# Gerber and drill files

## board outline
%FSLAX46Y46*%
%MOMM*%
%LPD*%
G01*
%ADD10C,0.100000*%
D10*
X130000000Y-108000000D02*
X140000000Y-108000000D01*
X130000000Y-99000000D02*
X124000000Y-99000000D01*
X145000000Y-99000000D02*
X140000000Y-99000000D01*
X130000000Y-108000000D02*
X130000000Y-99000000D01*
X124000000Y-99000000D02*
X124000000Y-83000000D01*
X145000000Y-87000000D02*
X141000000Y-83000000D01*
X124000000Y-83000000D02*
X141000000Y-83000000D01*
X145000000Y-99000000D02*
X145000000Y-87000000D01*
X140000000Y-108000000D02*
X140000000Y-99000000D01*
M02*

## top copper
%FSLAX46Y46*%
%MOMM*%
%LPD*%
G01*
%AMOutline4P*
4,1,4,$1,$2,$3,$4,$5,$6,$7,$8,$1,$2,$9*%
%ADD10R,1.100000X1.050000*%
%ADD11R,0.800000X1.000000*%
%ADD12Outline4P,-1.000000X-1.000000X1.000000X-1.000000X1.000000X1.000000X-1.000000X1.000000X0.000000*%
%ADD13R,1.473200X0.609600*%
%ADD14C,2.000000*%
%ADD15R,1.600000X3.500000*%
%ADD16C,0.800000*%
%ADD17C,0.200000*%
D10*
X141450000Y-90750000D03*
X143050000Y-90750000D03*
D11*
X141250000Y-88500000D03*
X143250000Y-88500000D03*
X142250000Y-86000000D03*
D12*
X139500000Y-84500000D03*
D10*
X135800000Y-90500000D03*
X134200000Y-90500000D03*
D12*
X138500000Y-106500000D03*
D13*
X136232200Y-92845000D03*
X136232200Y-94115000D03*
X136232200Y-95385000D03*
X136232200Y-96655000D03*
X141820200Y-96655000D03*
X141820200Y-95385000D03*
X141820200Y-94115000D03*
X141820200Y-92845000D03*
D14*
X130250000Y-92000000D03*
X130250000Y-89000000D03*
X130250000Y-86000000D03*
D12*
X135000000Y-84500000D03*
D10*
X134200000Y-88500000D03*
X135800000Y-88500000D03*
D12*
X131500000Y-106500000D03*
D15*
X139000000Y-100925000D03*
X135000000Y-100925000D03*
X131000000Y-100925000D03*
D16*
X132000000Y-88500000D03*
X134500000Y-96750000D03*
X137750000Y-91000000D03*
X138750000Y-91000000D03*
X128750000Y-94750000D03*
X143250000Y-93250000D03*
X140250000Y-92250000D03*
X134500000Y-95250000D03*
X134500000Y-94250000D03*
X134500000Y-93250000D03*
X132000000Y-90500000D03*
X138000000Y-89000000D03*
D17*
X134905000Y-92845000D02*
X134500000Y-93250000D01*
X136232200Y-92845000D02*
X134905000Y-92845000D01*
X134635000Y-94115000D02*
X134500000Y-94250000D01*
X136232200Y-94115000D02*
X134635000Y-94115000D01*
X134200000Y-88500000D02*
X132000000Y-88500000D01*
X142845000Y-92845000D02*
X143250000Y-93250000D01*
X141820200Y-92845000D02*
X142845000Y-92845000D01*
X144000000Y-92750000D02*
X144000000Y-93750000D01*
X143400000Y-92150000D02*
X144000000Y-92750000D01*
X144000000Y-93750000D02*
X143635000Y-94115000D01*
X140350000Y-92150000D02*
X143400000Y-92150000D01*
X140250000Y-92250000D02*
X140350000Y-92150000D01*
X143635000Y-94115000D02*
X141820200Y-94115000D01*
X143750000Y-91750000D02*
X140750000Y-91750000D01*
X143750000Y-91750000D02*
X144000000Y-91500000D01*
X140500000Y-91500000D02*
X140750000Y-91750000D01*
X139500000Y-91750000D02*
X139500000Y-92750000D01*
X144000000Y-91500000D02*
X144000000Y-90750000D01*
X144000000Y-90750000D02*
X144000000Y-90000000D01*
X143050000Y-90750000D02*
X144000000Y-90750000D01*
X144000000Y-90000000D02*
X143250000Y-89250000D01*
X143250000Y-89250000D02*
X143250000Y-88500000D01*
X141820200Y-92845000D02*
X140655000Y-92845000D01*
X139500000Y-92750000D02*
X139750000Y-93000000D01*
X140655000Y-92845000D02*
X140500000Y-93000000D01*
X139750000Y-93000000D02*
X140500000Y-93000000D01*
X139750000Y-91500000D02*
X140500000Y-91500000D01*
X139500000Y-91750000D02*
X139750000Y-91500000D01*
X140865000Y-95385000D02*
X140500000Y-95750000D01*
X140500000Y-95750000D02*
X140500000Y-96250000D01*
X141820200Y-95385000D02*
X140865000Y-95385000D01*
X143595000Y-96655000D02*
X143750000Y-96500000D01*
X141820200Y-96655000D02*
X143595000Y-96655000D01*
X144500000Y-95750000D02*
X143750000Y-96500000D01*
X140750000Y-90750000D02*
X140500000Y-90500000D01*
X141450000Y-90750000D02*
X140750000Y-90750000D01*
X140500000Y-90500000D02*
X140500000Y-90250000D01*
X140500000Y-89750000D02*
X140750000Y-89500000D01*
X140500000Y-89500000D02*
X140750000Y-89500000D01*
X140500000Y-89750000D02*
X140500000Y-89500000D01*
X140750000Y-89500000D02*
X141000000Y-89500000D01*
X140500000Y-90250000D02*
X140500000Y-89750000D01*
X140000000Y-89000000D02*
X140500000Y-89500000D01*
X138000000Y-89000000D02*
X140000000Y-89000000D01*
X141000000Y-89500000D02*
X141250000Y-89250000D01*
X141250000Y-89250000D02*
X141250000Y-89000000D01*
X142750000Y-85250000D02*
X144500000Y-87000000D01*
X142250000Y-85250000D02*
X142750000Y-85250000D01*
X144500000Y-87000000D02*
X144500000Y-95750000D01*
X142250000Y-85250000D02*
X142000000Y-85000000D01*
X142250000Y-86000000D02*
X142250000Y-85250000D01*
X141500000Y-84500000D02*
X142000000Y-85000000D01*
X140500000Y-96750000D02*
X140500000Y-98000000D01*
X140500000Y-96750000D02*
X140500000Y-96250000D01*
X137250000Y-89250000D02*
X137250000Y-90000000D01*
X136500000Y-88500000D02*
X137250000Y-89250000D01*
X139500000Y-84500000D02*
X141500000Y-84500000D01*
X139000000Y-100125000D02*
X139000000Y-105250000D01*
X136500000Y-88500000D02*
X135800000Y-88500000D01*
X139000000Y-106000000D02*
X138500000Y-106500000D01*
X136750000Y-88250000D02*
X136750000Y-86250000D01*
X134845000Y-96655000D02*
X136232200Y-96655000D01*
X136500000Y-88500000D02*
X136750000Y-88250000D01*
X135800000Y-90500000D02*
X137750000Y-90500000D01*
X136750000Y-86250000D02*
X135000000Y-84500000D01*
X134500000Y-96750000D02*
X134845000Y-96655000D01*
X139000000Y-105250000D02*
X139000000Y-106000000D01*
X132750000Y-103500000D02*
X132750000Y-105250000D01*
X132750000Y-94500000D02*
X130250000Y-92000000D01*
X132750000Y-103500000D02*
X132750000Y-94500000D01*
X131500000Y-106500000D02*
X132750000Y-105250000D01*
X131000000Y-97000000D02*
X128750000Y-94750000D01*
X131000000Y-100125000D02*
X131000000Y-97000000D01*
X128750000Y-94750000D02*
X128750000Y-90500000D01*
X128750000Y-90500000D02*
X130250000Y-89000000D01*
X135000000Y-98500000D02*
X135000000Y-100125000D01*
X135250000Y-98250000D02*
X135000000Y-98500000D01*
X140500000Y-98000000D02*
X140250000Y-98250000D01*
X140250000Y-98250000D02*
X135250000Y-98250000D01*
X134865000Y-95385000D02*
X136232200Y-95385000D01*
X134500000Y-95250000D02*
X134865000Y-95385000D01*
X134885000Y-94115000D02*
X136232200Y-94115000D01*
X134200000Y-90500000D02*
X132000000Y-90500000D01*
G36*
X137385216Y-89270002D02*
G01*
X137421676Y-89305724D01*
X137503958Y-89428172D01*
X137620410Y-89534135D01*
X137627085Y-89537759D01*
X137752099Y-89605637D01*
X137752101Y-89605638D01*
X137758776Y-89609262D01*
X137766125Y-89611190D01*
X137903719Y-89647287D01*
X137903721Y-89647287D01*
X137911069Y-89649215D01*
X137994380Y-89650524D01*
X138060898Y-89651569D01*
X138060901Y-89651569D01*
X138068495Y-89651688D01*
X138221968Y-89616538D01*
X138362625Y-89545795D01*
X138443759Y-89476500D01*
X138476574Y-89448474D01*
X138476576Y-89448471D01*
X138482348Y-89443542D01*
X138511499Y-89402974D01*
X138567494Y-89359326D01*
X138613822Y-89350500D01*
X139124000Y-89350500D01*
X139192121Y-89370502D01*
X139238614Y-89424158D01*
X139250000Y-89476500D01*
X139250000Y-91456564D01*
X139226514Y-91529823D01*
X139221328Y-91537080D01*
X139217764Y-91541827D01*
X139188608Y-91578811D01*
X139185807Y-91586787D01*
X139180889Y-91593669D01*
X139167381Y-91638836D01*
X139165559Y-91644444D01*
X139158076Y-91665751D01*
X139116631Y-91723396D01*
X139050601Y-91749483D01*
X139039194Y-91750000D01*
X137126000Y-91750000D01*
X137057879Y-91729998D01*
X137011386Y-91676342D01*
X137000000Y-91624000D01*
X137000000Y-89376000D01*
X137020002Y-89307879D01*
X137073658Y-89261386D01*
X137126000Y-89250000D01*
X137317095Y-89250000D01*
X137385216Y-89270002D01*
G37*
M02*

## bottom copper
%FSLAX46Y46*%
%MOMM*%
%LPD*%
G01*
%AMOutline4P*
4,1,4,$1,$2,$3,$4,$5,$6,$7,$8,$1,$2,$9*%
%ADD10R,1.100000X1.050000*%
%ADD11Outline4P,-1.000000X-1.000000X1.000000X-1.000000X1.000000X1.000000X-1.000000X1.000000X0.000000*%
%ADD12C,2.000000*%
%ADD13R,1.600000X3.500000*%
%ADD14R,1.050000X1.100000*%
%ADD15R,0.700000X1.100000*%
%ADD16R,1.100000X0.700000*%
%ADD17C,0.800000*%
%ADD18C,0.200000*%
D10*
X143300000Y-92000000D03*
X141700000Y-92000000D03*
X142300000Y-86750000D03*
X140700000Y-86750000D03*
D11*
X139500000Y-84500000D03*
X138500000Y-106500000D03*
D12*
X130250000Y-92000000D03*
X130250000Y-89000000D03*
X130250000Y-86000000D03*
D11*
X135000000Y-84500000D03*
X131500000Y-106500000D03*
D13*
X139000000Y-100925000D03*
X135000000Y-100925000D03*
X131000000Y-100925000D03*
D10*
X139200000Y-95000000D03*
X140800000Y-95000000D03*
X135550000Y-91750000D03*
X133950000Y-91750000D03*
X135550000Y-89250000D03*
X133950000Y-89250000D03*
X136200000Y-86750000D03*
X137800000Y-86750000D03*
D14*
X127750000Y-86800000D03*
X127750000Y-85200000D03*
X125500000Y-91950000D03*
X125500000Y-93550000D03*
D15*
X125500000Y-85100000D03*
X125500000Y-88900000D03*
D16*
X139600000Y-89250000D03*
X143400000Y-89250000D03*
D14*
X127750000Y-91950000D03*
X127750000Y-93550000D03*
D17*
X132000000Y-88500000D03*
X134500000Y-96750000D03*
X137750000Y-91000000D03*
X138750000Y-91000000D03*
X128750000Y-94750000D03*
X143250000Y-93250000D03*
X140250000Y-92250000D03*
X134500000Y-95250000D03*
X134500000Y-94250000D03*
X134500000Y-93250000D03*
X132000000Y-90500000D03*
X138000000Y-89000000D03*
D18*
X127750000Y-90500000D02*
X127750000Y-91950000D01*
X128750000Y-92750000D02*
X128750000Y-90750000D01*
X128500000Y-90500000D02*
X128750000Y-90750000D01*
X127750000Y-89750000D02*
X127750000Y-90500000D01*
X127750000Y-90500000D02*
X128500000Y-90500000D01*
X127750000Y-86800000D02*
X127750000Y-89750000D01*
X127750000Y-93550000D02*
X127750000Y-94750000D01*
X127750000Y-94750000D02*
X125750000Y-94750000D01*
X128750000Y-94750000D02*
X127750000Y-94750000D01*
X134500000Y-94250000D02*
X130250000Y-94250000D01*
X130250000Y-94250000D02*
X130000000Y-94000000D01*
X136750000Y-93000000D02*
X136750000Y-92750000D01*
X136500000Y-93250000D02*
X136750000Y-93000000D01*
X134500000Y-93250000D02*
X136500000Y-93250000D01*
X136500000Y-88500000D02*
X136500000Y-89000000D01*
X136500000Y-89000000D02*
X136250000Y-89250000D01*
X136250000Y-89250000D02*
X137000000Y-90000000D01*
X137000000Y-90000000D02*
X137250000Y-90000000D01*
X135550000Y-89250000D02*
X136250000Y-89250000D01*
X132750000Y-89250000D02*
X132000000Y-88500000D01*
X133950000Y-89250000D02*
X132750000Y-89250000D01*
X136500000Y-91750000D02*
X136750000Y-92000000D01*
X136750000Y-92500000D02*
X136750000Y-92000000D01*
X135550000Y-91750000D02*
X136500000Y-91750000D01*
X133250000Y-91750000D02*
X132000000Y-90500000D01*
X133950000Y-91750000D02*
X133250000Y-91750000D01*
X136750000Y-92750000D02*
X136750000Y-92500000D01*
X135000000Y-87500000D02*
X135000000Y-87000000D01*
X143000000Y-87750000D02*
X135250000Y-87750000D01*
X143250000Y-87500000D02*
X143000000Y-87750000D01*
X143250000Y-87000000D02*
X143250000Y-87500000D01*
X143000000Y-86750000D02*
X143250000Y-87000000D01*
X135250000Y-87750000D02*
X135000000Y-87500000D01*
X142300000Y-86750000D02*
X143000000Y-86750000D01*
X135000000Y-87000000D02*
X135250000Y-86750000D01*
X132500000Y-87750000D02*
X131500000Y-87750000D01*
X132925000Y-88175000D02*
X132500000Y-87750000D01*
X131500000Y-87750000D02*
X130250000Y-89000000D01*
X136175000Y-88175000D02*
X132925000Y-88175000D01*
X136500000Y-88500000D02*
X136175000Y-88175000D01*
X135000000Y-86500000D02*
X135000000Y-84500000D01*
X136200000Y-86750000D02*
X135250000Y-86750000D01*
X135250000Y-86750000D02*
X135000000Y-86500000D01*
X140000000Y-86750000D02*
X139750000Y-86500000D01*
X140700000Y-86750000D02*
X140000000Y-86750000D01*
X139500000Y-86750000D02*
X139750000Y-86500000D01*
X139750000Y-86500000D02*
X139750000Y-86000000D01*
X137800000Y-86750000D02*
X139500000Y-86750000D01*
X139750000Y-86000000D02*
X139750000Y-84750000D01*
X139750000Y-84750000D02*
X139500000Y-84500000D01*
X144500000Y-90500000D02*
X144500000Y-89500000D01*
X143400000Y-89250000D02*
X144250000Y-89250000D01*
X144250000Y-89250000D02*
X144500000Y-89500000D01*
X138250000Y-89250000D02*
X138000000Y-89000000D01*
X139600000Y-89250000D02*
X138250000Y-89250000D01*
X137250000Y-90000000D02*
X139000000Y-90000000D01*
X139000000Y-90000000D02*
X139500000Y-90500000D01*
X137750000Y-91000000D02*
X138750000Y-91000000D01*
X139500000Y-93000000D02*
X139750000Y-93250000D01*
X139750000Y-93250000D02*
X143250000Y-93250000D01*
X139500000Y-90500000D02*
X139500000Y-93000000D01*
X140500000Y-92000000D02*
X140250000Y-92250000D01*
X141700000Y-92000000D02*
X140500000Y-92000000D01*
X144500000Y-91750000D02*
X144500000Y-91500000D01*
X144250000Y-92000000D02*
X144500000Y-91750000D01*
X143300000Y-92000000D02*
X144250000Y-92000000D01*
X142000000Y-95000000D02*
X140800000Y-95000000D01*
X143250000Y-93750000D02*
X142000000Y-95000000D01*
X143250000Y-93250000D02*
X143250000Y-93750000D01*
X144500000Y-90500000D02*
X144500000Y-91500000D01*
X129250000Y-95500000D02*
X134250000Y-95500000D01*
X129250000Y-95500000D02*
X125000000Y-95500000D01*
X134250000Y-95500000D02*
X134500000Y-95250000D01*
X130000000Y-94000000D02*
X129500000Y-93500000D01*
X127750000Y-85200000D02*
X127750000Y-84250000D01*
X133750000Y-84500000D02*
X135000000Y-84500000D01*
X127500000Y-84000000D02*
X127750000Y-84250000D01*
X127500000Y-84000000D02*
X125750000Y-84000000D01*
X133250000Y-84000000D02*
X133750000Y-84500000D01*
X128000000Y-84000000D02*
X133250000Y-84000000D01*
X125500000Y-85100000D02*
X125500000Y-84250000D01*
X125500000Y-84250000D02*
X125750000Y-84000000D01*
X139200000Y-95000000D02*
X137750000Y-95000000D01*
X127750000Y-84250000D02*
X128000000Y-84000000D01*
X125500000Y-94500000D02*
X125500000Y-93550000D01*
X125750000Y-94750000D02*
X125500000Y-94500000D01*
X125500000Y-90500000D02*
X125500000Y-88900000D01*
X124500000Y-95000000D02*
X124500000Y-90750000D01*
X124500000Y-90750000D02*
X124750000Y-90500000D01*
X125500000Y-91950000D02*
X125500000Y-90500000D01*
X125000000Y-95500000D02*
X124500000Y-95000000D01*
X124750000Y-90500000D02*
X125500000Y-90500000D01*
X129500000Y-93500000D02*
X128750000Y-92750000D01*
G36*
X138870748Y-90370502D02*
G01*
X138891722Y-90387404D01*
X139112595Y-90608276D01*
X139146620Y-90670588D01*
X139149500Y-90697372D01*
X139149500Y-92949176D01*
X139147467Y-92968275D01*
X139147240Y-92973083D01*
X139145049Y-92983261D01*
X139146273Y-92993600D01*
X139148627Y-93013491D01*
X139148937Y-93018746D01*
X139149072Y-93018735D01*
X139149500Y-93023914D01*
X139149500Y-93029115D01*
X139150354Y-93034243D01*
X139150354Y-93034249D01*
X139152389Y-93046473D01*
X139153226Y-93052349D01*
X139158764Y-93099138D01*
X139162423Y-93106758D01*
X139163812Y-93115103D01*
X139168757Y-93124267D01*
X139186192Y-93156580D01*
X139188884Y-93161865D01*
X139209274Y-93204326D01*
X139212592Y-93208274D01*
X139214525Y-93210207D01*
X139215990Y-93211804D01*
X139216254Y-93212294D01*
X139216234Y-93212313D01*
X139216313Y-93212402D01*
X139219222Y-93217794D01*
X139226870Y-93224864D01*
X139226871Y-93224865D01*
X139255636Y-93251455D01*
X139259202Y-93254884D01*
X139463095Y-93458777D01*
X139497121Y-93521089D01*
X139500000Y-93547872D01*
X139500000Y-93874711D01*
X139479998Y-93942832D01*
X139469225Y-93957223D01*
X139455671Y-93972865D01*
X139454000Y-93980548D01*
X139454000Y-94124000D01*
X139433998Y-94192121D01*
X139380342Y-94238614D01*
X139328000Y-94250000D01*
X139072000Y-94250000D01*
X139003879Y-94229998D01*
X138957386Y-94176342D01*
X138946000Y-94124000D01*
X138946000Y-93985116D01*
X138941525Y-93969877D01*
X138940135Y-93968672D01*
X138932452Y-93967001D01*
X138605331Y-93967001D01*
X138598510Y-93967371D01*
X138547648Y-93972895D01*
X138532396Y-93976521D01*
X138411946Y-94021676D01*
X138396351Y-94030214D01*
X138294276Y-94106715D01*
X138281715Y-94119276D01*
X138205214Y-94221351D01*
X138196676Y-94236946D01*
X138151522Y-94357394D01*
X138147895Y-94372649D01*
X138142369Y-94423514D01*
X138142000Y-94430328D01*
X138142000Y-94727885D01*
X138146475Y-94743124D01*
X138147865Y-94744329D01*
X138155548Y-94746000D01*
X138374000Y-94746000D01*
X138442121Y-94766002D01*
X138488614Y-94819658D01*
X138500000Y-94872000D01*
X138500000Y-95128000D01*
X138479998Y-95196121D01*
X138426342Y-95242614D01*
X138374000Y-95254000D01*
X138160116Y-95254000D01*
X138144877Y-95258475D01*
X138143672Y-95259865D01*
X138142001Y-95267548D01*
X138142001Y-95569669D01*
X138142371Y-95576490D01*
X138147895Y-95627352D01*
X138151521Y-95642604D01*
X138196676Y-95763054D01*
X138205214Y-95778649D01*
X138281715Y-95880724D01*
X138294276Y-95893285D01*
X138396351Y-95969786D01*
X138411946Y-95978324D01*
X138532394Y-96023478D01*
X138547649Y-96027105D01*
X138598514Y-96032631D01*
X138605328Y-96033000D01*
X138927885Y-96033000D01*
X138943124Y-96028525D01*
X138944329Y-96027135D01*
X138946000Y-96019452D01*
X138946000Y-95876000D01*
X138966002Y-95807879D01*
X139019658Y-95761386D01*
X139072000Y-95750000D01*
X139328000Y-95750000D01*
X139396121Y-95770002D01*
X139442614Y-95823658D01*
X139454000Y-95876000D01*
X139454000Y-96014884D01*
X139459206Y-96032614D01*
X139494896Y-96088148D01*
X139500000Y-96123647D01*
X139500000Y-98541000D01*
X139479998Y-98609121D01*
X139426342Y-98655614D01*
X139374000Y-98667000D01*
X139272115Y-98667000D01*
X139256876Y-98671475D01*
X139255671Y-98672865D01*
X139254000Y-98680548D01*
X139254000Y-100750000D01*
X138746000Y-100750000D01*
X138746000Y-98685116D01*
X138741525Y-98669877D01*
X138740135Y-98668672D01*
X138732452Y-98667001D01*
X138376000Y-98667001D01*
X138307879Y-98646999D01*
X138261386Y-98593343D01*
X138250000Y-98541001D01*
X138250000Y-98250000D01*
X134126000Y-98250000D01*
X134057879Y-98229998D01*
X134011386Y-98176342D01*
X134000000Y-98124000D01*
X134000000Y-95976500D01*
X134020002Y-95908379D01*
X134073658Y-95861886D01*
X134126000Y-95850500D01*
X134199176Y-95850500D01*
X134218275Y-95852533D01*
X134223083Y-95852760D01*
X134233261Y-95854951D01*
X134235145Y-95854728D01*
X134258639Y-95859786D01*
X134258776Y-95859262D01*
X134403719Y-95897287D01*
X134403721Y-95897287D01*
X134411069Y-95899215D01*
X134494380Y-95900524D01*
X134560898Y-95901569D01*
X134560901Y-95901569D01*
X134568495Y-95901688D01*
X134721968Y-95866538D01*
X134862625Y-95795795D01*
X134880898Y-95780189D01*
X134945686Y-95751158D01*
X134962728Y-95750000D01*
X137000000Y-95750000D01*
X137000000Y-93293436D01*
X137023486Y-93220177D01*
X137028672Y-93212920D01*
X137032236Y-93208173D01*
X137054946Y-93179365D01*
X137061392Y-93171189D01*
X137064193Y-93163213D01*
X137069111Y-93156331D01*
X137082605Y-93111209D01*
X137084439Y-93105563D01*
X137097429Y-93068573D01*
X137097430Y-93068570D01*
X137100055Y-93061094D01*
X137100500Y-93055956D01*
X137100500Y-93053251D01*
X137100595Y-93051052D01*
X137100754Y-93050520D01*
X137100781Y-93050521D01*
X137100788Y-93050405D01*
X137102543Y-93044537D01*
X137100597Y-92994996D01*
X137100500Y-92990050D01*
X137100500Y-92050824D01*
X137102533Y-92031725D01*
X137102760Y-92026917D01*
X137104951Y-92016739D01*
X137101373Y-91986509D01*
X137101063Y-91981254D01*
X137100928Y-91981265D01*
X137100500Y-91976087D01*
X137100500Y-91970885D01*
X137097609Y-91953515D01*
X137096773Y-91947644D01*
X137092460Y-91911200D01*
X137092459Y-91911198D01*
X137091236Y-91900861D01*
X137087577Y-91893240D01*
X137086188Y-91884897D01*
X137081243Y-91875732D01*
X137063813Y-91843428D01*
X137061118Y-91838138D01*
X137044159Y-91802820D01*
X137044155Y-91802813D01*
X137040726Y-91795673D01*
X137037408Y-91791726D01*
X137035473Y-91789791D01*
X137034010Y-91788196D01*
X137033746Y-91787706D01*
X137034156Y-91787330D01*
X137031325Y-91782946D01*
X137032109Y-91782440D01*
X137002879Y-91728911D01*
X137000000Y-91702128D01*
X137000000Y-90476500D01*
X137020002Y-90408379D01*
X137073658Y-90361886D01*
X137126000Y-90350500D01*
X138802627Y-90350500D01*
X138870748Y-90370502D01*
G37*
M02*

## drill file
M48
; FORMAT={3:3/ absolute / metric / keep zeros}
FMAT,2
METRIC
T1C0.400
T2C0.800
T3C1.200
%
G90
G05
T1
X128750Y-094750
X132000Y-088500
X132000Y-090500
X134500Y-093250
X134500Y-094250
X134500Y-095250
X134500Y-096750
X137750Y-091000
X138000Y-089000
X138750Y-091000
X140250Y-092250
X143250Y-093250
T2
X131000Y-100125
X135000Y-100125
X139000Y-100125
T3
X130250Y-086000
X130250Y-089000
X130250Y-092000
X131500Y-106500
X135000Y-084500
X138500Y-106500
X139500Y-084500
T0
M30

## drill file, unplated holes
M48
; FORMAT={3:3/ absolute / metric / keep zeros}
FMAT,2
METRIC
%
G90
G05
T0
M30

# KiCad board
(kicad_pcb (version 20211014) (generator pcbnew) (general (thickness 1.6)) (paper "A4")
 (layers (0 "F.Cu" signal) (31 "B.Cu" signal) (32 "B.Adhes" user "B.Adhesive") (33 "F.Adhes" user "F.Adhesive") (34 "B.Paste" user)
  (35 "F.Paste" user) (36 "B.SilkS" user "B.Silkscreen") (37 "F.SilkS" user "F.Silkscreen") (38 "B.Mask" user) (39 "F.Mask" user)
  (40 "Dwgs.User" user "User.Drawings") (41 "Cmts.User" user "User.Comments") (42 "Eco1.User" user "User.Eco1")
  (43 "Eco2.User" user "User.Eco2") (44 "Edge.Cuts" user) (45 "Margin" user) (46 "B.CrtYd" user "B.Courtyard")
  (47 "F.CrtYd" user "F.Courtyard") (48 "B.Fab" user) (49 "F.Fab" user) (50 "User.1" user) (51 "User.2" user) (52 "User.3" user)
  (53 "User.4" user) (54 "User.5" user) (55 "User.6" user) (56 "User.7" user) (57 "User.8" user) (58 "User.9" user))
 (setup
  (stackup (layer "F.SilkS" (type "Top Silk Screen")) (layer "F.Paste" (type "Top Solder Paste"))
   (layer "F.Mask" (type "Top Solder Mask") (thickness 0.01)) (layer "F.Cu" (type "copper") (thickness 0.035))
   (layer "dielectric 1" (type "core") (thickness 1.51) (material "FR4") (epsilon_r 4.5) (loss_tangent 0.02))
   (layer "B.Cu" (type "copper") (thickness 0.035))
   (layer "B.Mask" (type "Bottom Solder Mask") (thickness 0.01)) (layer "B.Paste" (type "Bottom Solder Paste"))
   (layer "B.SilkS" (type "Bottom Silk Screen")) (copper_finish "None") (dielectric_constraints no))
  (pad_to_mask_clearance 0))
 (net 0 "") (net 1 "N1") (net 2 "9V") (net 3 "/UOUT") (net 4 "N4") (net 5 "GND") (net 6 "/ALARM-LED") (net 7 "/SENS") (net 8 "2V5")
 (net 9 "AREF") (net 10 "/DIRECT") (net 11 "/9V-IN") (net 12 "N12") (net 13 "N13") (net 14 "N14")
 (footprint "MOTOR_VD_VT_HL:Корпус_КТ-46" (layer "F.Cu") (at 142.25 87.25 90)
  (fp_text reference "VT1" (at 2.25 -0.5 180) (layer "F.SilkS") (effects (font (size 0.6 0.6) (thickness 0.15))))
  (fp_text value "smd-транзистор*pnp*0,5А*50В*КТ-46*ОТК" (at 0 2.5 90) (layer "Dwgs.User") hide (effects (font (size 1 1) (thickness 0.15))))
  (pad "1" smd rect locked (at -1.25 -1 90) (size 1 0.8) (layers "F.Cu" "F.Paste" "F.Mask") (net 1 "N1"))
  (pad "2" smd rect locked (at -1.25 1 90) (size 1 0.8) (layers "F.Cu" "F.Paste" "F.Mask") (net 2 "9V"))
  (pad "3" smd rect locked (at 1.25 0 90) (size 1 0.8) (layers "F.Cu" "F.Paste" "F.Mask") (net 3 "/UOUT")))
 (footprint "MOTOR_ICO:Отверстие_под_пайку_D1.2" (layer "F.Cu") (at 139.5 84.5)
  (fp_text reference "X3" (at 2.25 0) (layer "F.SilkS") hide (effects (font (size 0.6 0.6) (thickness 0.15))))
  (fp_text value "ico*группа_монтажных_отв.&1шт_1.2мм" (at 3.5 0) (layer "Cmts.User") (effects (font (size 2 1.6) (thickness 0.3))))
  (pad "1" thru_hole trapezoid locked (at 0 0) (size 2 2) (drill 1.2) (layers *.Cu *.Paste *.Mask) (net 3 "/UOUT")))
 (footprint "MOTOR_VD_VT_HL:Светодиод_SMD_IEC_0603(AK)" (layer "F.Cu") (at 135 90.5)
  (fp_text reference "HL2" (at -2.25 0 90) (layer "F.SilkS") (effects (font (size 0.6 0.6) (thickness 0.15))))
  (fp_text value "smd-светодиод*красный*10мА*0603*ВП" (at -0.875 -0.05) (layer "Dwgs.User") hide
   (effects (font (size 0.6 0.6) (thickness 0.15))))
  (pad "A" smd rect locked (at -0.8 0) (size 1.1 1.05) (layers "F.Cu" "F.Paste" "F.Mask") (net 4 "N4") (clearance 0.2))
  (pad "K" smd rect locked (at 0.8 0) (size 1.1 1.05) (layers "F.Cu" "F.Paste" "F.Mask") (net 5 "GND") (clearance 0.2)))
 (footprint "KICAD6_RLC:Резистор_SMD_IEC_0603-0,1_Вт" (layer "F.Cu") (at 142.25 90.75)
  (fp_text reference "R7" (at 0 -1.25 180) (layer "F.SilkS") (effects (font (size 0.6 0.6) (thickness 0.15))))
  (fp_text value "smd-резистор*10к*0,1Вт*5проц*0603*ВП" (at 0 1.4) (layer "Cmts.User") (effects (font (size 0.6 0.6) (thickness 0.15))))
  (pad "1" smd rect (at -0.8 0) (size 1.1 1.05) (layers "F.Cu" "F.Paste" "F.Mask") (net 1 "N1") (clearance 0.2))
  (pad "2" smd rect (at 0.8 0) (size 1.1 1.05) (layers "F.Cu" "F.Paste" "F.Mask") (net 2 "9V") (clearance 0.2)))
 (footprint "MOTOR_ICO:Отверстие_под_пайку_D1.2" (layer "F.Cu") (at 138.5 106.5)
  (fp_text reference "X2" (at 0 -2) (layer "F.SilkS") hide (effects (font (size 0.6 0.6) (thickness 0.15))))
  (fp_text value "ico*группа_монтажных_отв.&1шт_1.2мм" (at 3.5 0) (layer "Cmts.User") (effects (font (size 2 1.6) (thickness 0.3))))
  (pad "1" thru_hole trapezoid locked (at 0 0) (size 2 2) (drill 1.2) (layers *.Cu *.Paste *.Mask) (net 5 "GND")))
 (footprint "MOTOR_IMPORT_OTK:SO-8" (layer "F.Cu") (at 136.2682 92.861 -90)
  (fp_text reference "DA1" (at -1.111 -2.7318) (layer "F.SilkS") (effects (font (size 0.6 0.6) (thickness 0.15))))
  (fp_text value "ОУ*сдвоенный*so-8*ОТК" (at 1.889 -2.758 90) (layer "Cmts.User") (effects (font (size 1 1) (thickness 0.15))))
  (pad "1" smd rect locked (at -0.016 0.036 270) (size 0.6096 1.4732) (layers "F.Cu" "F.Paste" "F.Mask") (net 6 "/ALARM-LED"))
  (pad "2" smd rect locked (at 1.254 0.036 270) (size 0.6096 1.4732) (layers "F.Cu" "F.Paste" "F.Mask") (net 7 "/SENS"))
  (pad "3" smd rect locked (at 2.524 0.036 270) (size 0.6096 1.4732) (layers "F.Cu" "F.Paste" "F.Mask") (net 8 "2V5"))
  (pad "4" smd rect locked (at 3.794 0.036 270) (size 0.6096 1.4732) (layers "F.Cu" "F.Paste" "F.Mask") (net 5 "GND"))
  (pad "5" smd rect locked (at 3.794 -5.552 270) (size 0.6096 1.4732) (layers "F.Cu" "F.Paste" "F.Mask") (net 3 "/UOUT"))
  (pad "6" smd rect locked (at 2.524 -5.552 270) (size 0.6096 1.4732) (layers "F.Cu" "F.Paste" "F.Mask") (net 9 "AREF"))
  (pad "7" smd rect locked (at 1.254 -5.552 270) (size 0.6096 1.4732) (layers "F.Cu" "F.Paste" "F.Mask") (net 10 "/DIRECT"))
  (pad "8" smd rect locked (at -0.016 -5.552 270) (size 0.6096 1.4732) (layers "F.Cu" "F.Paste" "F.Mask") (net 2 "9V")))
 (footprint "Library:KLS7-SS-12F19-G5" (layer "F.Cu") (at 130.25 92 90)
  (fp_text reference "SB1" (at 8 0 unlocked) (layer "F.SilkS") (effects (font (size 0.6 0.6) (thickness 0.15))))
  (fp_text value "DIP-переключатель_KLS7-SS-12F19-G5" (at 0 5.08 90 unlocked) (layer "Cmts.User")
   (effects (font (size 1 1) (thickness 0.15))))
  (pad "1" thru_hole circle (at 0 0 90) (size 2 2) (drill 1.2) (layers *.Cu *.Mask) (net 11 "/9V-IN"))
  (pad "2" thru_hole circle (at 3 0 90) (size 2 2) (drill 1.2) (layers *.Cu *.Mask) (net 2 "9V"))
  (pad "3" thru_hole circle (at 6 0 90) (size 2 2) (drill 1.2) (layers *.Cu *.Mask) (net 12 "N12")))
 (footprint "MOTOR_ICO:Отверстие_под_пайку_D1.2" (layer "F.Cu") (at 135 84.5)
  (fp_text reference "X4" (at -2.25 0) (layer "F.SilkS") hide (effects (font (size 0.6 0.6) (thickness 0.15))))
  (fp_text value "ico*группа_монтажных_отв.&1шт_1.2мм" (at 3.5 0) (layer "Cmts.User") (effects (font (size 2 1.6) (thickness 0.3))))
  (pad "1" thru_hole trapezoid locked (at 0 0) (size 2 2) (drill 1.2) (layers *.Cu *.Paste *.Mask) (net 5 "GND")))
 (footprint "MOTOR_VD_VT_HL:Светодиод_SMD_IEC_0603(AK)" (layer "F.Cu") (at 135 88.5)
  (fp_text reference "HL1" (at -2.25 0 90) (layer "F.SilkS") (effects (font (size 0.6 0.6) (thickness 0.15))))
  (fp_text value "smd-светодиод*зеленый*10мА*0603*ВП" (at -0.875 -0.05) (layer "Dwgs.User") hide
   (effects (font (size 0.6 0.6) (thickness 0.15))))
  (pad "A" smd rect locked (at -0.8 0) (size 1.1 1.05) (layers "F.Cu" "F.Paste" "F.Mask") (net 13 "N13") (clearance 0.2))
  (pad "K" smd rect locked (at 0.8 0) (size 1.1 1.05) (layers "F.Cu" "F.Paste" "F.Mask") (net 5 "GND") (clearance 0.2)))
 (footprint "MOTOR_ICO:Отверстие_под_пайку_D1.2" (layer "F.Cu") (at 131.5 106.5)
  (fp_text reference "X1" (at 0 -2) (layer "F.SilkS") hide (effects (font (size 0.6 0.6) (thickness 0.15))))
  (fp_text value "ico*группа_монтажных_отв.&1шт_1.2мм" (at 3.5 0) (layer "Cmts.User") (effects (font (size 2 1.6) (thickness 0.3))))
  (pad "1" thru_hole trapezoid locked (at 0 0) (size 2 2) (drill 1.2) (layers *.Cu *.Paste *.Mask) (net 11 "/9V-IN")))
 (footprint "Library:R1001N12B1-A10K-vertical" (layer "F.Cu") (at 139 100.125 180)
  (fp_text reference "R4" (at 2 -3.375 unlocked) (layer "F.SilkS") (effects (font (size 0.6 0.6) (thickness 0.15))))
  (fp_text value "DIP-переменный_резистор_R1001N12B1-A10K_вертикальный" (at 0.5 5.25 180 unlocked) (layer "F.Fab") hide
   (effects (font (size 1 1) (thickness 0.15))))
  (pad "1" thru_hole rect (at 0 0 180) (size 1.6 3.5) (drill 0.8 (offset 0 -0.8)) (layers *.Cu *.Mask) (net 5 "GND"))
  (pad "2" thru_hole rect (at 4 0 180) (size 1.6 3.5) (drill 0.8 (offset 0 -0.8)) (layers *.Cu *.Mask) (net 9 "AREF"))
  (pad "3" thru_hole rect (at 8 0 180) (size 1.6 3.5) (drill 0.8 (offset 0 -0.8)) (layers *.Cu *.Mask) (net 2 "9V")))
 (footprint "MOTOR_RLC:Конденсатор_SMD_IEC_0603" (layer "B.Cu") (at 140 95)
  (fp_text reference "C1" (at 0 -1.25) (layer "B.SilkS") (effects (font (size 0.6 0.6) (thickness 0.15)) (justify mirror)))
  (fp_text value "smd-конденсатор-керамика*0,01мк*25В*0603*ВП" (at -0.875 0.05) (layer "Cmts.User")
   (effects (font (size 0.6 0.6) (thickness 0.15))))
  (pad "1" smd rect locked (at -0.8 0) (size 1.1 1.05) (layers "B.Cu" "B.Paste" "B.Mask") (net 5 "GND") (clearance 0.2))
  (pad "2" smd rect locked (at 0.8 0) (size 1.1 1.05) (layers "B.Cu" "B.Paste" "B.Mask") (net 2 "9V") (clearance 0.2)))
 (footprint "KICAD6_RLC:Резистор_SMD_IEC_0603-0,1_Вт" (layer "B.Cu") (at 134.75 91.75 180)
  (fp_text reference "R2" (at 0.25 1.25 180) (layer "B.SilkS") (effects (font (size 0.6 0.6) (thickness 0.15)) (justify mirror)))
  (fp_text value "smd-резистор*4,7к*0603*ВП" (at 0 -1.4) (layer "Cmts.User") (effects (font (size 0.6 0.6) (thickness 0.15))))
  (pad "1" smd rect (at -0.8 0 180) (size 1.1 1.05) (layers "B.Cu" "B.Paste" "B.Mask") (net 6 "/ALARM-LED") (clearance 0.2))
  (pad "2" smd rect (at 0.8 0 180) (size 1.1 1.05) (layers "B.Cu" "B.Paste" "B.Mask") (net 4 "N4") (clearance 0.2)))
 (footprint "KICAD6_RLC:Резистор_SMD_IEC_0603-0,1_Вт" (layer "B.Cu") (at 134.75 89.25 180)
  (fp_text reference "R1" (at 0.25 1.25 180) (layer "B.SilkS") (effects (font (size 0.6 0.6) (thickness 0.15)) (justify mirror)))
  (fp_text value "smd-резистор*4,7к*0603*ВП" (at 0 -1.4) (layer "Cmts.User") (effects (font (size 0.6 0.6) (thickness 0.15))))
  (pad "1" smd rect (at -0.8 0 180) (size 1.1 1.05) (layers "B.Cu" "B.Paste" "B.Mask") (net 2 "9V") (clearance 0.2))
  (pad "2" smd rect (at 0.8 0 180) (size 1.1 1.05) (layers "B.Cu" "B.Paste" "B.Mask") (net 13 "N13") (clearance 0.2)))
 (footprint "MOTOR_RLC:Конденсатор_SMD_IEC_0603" (layer "B.Cu") (at 137 86.75)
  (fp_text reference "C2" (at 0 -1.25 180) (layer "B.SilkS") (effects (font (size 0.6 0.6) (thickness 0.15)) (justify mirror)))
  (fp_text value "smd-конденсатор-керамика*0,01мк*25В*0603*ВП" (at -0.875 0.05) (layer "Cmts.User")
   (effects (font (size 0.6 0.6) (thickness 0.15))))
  (pad "1" smd rect locked (at -0.8 0) (size 1.1 1.05) (layers "B.Cu" "B.Paste" "B.Mask") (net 5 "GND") (clearance 0.2))
  (pad "2" smd rect locked (at 0.8 0) (size 1.1 1.05) (layers "B.Cu" "B.Paste" "B.Mask") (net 3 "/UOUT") (clearance 0.2)))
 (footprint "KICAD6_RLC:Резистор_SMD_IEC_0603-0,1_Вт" (layer "B.Cu") (at 127.75 86 -90)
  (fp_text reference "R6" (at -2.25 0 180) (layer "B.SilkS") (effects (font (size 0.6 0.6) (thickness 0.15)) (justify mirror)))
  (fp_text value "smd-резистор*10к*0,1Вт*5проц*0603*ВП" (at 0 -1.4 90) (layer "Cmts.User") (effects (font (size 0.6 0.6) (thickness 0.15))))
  (pad "1" smd rect (at -0.8 0 270) (size 1.1 1.05) (layers "B.Cu" "B.Paste" "B.Mask") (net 5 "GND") (clearance 0.2))
  (pad "2" smd rect (at 0.8 0 270) (size 1.1 1.05) (layers "B.Cu" "B.Paste" "B.Mask") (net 7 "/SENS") (clearance 0.2)))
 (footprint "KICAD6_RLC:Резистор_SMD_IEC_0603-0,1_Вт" (layer "B.Cu") (at 142.5 92 180)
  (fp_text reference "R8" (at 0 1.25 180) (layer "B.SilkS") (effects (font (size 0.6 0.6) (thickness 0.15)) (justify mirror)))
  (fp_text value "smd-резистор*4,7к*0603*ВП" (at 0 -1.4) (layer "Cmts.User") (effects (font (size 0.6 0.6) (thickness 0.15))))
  (pad "1" smd rect (at -0.8 0 180) (size 1.1 1.05) (layers "B.Cu" "B.Paste" "B.Mask") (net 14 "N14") (clearance 0.2))
  (pad "2" smd rect (at 0.8 0 180) (size 1.1 1.05) (layers "B.Cu" "B.Paste" "B.Mask") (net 10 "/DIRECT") (clearance 0.2)))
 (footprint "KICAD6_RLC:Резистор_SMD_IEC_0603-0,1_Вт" (layer "B.Cu") (at 125.5 92.75 -90)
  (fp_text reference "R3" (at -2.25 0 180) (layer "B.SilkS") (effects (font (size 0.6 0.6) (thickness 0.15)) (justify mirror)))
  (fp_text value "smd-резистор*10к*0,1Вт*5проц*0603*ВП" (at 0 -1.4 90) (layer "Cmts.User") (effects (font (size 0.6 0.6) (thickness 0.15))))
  (pad "1" smd rect (at -0.8 0 270) (size 1.1 1.05) (layers "B.Cu" "B.Paste" "B.Mask") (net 8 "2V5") (clearance 0.2))
  (pad "2" smd rect (at 0.8 0 270) (size 1.1 1.05) (layers "B.Cu" "B.Paste" "B.Mask") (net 2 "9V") (clearance 0.2)))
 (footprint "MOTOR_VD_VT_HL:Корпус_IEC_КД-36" (layer "B.Cu") (at 125.5 87 90)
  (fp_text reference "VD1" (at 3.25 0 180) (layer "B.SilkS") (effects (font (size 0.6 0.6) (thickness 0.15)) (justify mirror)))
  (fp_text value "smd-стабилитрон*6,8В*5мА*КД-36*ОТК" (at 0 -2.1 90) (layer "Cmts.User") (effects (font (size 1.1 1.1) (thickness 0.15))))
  (pad "A" smd rect locked (at 1.9 0 90) (size 1.1 0.7) (layers "B.Cu" "B.Paste" "B.Mask") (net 5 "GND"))
  (pad "K" smd rect locked (at -1.9 0 90) (size 1.1 0.7) (layers "B.Cu" "B.Paste" "B.Mask") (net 8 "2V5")))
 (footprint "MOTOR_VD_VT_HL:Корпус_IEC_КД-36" (layer "B.Cu") (at 141.5 89.25)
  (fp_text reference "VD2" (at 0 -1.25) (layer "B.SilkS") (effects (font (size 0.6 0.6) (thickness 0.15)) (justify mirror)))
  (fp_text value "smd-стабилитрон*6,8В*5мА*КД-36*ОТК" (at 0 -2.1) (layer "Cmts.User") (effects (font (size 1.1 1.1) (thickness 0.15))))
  (pad "A" smd rect locked (at 1.9 0) (size 1.1 0.7) (layers "B.Cu" "B.Paste" "B.Mask") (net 14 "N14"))
  (pad "K" smd rect locked (at -1.9 0) (size 1.1 0.7) (layers "B.Cu" "B.Paste" "B.Mask") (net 1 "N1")))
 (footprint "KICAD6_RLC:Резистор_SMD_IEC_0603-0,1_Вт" (layer "B.Cu") (at 141.5 86.75 180)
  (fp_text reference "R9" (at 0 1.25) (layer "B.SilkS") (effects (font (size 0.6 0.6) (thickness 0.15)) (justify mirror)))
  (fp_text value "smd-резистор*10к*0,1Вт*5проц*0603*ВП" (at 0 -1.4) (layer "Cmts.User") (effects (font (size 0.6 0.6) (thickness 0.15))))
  (pad "1" smd rect (at -0.8 0 180) (size 1.1 1.05) (layers "B.Cu" "B.Paste" "B.Mask") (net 5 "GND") (clearance 0.2))
  (pad "2" smd rect (at 0.8 0 180) (size 1.1 1.05) (layers "B.Cu" "B.Paste" "B.Mask") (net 3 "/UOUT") (clearance 0.2)))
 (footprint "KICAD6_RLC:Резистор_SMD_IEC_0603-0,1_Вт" (layer "B.Cu") (at 127.75 92.75 -90)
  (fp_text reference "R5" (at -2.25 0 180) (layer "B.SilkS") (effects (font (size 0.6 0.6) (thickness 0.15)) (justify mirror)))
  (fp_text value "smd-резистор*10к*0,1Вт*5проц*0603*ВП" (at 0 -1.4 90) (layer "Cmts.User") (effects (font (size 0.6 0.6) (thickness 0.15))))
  (pad "1" smd rect (at -0.8 0 270) (size 1.1 1.05) (layers "B.Cu" "B.Paste" "B.Mask") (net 7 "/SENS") (clearance 0.2))
  (pad "2" smd rect (at 0.8 0 270) (size 1.1 1.05) (layers "B.Cu" "B.Paste" "B.Mask") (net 2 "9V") (clearance 0.2)))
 (gr_line (start 130 108) (end 140 108) (layer "Edge.Cuts") (width 0.1))
 (gr_line (start 130 99) (end 124 99) (layer "Edge.Cuts") (width 0.1))
 (gr_line (start 145 99) (end 140 99) (layer "Edge.Cuts") (width 0.1))
 (gr_line (start 130 108) (end 130 99) (layer "Edge.Cuts") (width 0.1))
 (gr_line (start 124 99) (end 124 83) (layer "Edge.Cuts") (width 0.1))
 (gr_line (start 145 87) (end 141 83) (layer "Edge.Cuts") (width 0.1))
 (gr_line (start 124 83) (end 141 83) (layer "Edge.Cuts") (width 0.1))
 (gr_line (start 145 99) (end 145 87) (layer "Edge.Cuts") (width 0.1))
 (gr_line (start 140 108) (end 140 99) (layer "Edge.Cuts") (width 0.1))
 (segment (start 139 100.125) (end 139 105.25) (width 0.2) (layer "F.Cu") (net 5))
 (segment (start 136.5 88.5) (end 135.8 88.5) (width 0.2) (layer "F.Cu") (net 5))
 (segment (start 139 106) (end 138.5 106.5) (width 0.2) (layer "F.Cu") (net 5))
 (segment (start 136.75 88.25) (end 136.75 86.25) (width 0.2) (layer "F.Cu") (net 5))
 (segment (start 136.5 88.5) (end 137.25 89.25) (width 0.2) (layer "F.Cu") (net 5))
 (segment (start 134.845 96.655) (end 136.2322 96.655) (width 0.2) (layer "F.Cu") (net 5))
 (segment (start 136.5 88.5) (end 136.75 88.25) (width 0.2) (layer "F.Cu") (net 5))
 (segment (start 137.25 89.25) (end 137.25 90) (width 0.2) (layer "F.Cu") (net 5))
 (segment (start 135.8 90.5) (end 137.75 90.5) (width 0.2) (layer "F.Cu") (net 5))
 (segment (start 136.75 86.25) (end 135 84.5) (width 0.2) (layer "F.Cu") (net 5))
 (segment (start 134.5 96.75) (end 134.845 96.655) (width 0.2) (layer "F.Cu") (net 5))
 (segment (start 139 105.25) (end 139 106) (width 0.2) (layer "F.Cu") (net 5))
 (via (at 134.5 96.75) (size 0.8) (drill 0.4) (layers "F.Cu" "B.Cu") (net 5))
 (via (at 137.75 91) (size 0.8) (drill 0.4) (layers "F.Cu" "B.Cu") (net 5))
 (via (at 138.75 91) (size 0.8) (drill 0.4) (layers "F.Cu" "B.Cu") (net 5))
 (segment (start 127.75 85.2) (end 127.75 84.25) (width 0.2) (layer "B.Cu") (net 5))
 (segment (start 133.75 84.5) (end 135 84.5) (width 0.2) (layer "B.Cu") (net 5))
 (segment (start 143.25 87.5) (end 143 87.75) (width 0.2) (layer "B.Cu") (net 5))
 (segment (start 127.5 84) (end 127.75 84.25) (width 0.2) (layer "B.Cu") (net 5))
 (segment (start 143.25 87) (end 143.25 87.5) (width 0.2) (layer "B.Cu") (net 5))
 (segment (start 127.5 84) (end 125.75 84) (width 0.2) (layer "B.Cu") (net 5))
 (segment (start 135 87.5) (end 135 87) (width 0.2) (layer "B.Cu") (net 5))
 (segment (start 142.3 86.75) (end 143 86.75) (width 0.2) (layer "B.Cu") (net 5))
 (segment (start 133.25 84) (end 133.75 84.5) (width 0.2) (layer "B.Cu") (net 5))
 (segment (start 128 84) (end 133.25 84) (width 0.2) (layer "B.Cu") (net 5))
 (segment (start 136.2 86.75) (end 135.25 86.75) (width 0.2) (layer "B.Cu") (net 5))
 (segment (start 125.5 85.1) (end 125.5 84.25) (width 0.2) (layer "B.Cu") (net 5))
 (segment (start 143 86.75) (end 143.25 87) (width 0.2) (layer "B.Cu") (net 5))
 (segment (start 125.5 84.25) (end 125.75 84) (width 0.2) (layer "B.Cu") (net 5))
 (segment (start 139.2 95) (end 137.75 95) (width 0.2) (layer "B.Cu") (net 5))
 (segment (start 127.75 84.25) (end 128 84) (width 0.2) (layer "B.Cu") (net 5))
 (segment (start 135.25 86.75) (end 135 86.5) (width 0.2) (layer "B.Cu") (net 5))
 (segment (start 137.75 91) (end 138.75 91) (width 0.2) (layer "B.Cu") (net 5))
 (segment (start 135 86.5) (end 135 84.5) (width 0.2) (layer "B.Cu") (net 5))
 (segment (start 143 87.75) (end 135.25 87.75) (width 0.2) (layer "B.Cu") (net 5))
 (segment (start 135 87) (end 135.25 86.75) (width 0.2) (layer "B.Cu") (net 5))
 (segment (start 135.25 87.75) (end 135 87.5) (width 0.2) (layer "B.Cu") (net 5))
 (segment (start 132.75 103.5) (end 132.75 105.25) (width 0.2) (layer "F.Cu") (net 11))
 (segment (start 132.75 94.5) (end 130.25 92) (width 0.2) (layer "F.Cu") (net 11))
 (segment (start 132.75 103.5) (end 132.75 94.5) (width 0.2) (layer "F.Cu") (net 11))
 (segment (start 131.5 106.5) (end 132.75 105.25) (width 0.2) (layer "F.Cu") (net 11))
 (segment (start 134.2 88.5) (end 132 88.5) (width 0.2) (layer "F.Cu") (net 13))
 (via (at 132 88.5) (size 0.8) (drill 0.4) (layers "F.Cu" "B.Cu") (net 13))
 (segment (start 132.75 89.25) (end 132 88.5) (width 0.2) (layer "B.Cu") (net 13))
 (segment (start 133.95 89.25) (end 132.75 89.25) (width 0.2) (layer "B.Cu") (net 13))
 (segment (start 139.5 92.75) (end 139.75 93) (width 0.2) (layer "F.Cu") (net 2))
 (segment (start 131 97) (end 128.75 94.75) (width 0.2) (layer "F.Cu") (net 2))
 (segment (start 140.5 91.5) (end 140.75 91.75) (width 0.2) (layer "F.Cu") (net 2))
 (segment (start 139.5 91.75) (end 139.75 91.5) (width 0.2) (layer "F.Cu") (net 2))
 (segment (start 143.75 91.75) (end 144 91.5) (width 0.2) (layer "F.Cu") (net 2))
 (segment (start 144 91.5) (end 144 90.75) (width 0.2) (layer "F.Cu") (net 2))
 (segment (start 142.845 92.845) (end 143.25 93.25) (width 0.2) (layer "F.Cu") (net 2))
 (segment (start 139.75 91.5) (end 140.5 91.5) (width 0.2) (layer "F.Cu") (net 2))
 (segment (start 143.75 91.75) (end 140.75 91.75) (width 0.2) (layer "F.Cu") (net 2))
 (segment (start 131 100.125) (end 131 97) (width 0.2) (layer "F.Cu") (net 2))
 (segment (start 128.75 94.75) (end 128.75 90.5) (width 0.2) (layer "F.Cu") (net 2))
 (segment (start 140.655 92.845) (end 140.5 93) (width 0.2) (layer "F.Cu") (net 2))
 (segment (start 128.75 90.5) (end 130.25 89) (width 0.2) (layer "F.Cu") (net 2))
 (segment (start 143.25 89.25) (end 143.25 88.5) (width 0.2) (layer "F.Cu") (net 2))
 (segment (start 139.5 91.75) (end 139.5 92.75) (width 0.2) (layer "F.Cu") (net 2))
 (segment (start 141.8202 92.845) (end 140.655 92.845) (width 0.2) (layer "F.Cu") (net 2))
 (segment (start 139.75 93) (end 140.5 93) (width 0.2) (layer "F.Cu") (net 2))
 (segment (start 144 90) (end 143.25 89.25) (width 0.2) (layer "F.Cu") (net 2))
 (segment (start 143.05 90.75) (end 144 90.75) (width 0.2) (layer "F.Cu") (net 2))
 (segment (start 141.8202 92.845) (end 142.845 92.845) (width 0.2) (layer "F.Cu") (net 2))
 (segment (start 144 90.75) (end 144 90) (width 0.2) (layer "F.Cu") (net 2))
 (via (at 128.75 94.75) (size 0.8) (drill 0.4) (layers "F.Cu" "B.Cu") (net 2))
 (via (at 143.25 93.25) (size 0.8) (drill 0.4) (layers "F.Cu" "B.Cu") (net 2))
 (segment (start 139 90) (end 139.5 90.5) (width 0.2) (layer "B.Cu") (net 2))
 (segment (start 127.75 94.75) (end 125.75 94.75) (width 0.2) (layer "B.Cu") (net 2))
 (segment (start 125.5 94.5) (end 125.5 93.55) (width 0.2) (layer "B.Cu") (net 2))
 (segment (start 136.175 88.175) (end 132.925 88.175) (width 0.2) (layer "B.Cu") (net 2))
 (segment (start 125.75 94.75) (end 125.5 94.5) (width 0.2) (layer "B.Cu") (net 2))
 (segment (start 137 90) (end 137.25 90) (width 0.2) (layer "B.Cu") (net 2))
 (segment (start 136.25 89.25) (end 137 90) (width 0.2) (layer "B.Cu") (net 2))
 (segment (start 143.25 93.25) (end 143.25 93.75) (width 0.2) (layer "B.Cu") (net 2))
 (segment (start 132.925 88.175) (end 132.5 87.75) (width 0.2) (layer "B.Cu") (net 2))
 (segment (start 142 95) (end 140.8 95) (width 0.2) (layer "B.Cu") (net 2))
 (segment (start 139.75 93.25) (end 143.25 93.25) (width 0.2) (layer "B.Cu") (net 2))
 (segment (start 139.5 93) (end 139.75 93.25) (width 0.2) (layer "B.Cu") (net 2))
 (segment (start 136.5 88.5) (end 136.5 89) (width 0.2) (layer "B.Cu") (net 2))
 (segment (start 137.25 90) (end 139 90) (width 0.2) (layer "B.Cu") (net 2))
 (segment (start 128.75 94.75) (end 127.75 94.75) (width 0.2) (layer "B.Cu") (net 2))
 (segment (start 139.5 90.5) (end 139.5 93) (width 0.2) (layer "B.Cu") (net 2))
 (segment (start 135.55 89.25) (end 136.25 89.25) (width 0.2) (layer "B.Cu") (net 2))
 (segment (start 136.5 89) (end 136.25 89.25) (width 0.2) (layer "B.Cu") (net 2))
 (segment (start 143.25 93.75) (end 142 95) (width 0.2) (layer "B.Cu") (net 2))
 (segment (start 136.5 88.5) (end 136.175 88.175) (width 0.2) (layer "B.Cu") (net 2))
 (segment (start 132.5 87.75) (end 131.5 87.75) (width 0.2) (layer "B.Cu") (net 2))
 (segment (start 127.75 93.55) (end 127.75 94.75) (width 0.2) (layer "B.Cu") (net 2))
 (segment (start 131.5 87.75) (end 130.25 89) (width 0.2) (layer "B.Cu") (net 2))
 (segment (start 144.5 87) (end 144.5 95.75) (width 0.2) (layer "F.Cu") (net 3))
 (segment (start 139.5 84.5) (end 141.5 84.5) (width 0.2) (layer "F.Cu") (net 3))
 (segment (start 142.75 85.25) (end 144.5 87) (width 0.2) (layer "F.Cu") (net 3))
 (segment (start 142.25 86) (end 142.25 85.25) (width 0.2) (layer "F.Cu") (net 3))
 (segment (start 144.5 95.75) (end 143.75 96.5) (width 0.2) (layer "F.Cu") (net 3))
 (segment (start 141.5 84.5) (end 142 85) (width 0.2) (layer "F.Cu") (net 3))
 (segment (start 142.25 85.25) (end 142 85) (width 0.2) (layer "F.Cu") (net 3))
 (segment (start 142.25 85.25) (end 142.75 85.25) (width 0.2) (layer "F.Cu") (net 3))
 (segment (start 141.8202 96.655) (end 143.595 96.655) (width 0.2) (layer "F.Cu") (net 3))
 (segment (start 143.595 96.655) (end 143.75 96.5) (width 0.2) (layer "F.Cu") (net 3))
 (segment (start 140 86.75) (end 139.75 86.5) (width 0.2) (layer "B.Cu") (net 3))
 (segment (start 139.75 84.75) (end 139.5 84.5) (width 0.2) (layer "B.Cu") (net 3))
 (segment (start 139.5 86.75) (end 139.75 86.5) (width 0.2) (layer "B.Cu") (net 3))
 (segment (start 139.75 86.5) (end 139.75 86) (width 0.2) (layer "B.Cu") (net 3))
 (segment (start 139.75 86) (end 139.75 84.75) (width 0.2) (layer "B.Cu") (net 3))
 (segment (start 137.8 86.75) (end 139.5 86.75) (width 0.2) (layer "B.Cu") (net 3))
 (segment (start 140.7 86.75) (end 140 86.75) (width 0.2) (layer "B.Cu") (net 3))
 (segment (start 143.4 92.15) (end 144 92.75) (width 0.2) (layer "F.Cu") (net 10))
 (segment (start 143.635 94.115) (end 141.8202 94.115) (width 0.2) (layer "F.Cu") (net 10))
 (segment (start 140.35 92.15) (end 143.4 92.15) (width 0.2) (layer "F.Cu") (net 10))
 (segment (start 144 92.75) (end 144 93.75) (width 0.2) (layer "F.Cu") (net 10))
 (segment (start 144 93.75) (end 143.635 94.115) (width 0.2) (layer "F.Cu") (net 10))
 (segment (start 140.25 92.25) (end 140.35 92.15) (width 0.2) (layer "F.Cu") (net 10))
 (via (at 140.25 92.25) (size 0.8) (drill 0.4) (layers "F.Cu" "B.Cu") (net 10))
 (segment (start 140.5 92) (end 140.25 92.25) (width 0.2) (layer "B.Cu") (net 10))
 (segment (start 141.7 92) (end 140.5 92) (width 0.2) (layer "B.Cu") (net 10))
 (segment (start 140.5 96.75) (end 140.5 96.25) (width 0.2) (layer "F.Cu") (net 9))
 (segment (start 140.865 95.385) (end 140.5 95.75) (width 0.2) (layer "F.Cu") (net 9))
 (segment (start 135 98.5) (end 135 100.125) (width 0.2) (layer "F.Cu") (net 9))
 (segment (start 140.5 95.75) (end 140.5 96.25) (width 0.2) (layer "F.Cu") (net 9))
 (segment (start 135.25 98.25) (end 135 98.5) (width 0.2) (layer "F.Cu") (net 9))
 (segment (start 140.5 98) (end 140.25 98.25) (width 0.2) (layer "F.Cu") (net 9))
 (segment (start 141.8202 95.385) (end 140.865 95.385) (width 0.2) (layer "F.Cu") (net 9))
 (segment (start 140.25 98.25) (end 135.25 98.25) (width 0.2) (layer "F.Cu") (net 9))
 (segment (start 140.5 96.75) (end 140.5 98) (width 0.2) (layer "F.Cu") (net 9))
 (segment (start 134.865 95.385) (end 136.2322 95.385) (width 0.2) (layer "F.Cu") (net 8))
 (segment (start 134.5 95.25) (end 134.865 95.385) (width 0.2) (layer "F.Cu") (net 8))
 (via (at 134.5 95.25) (size 0.8) (drill 0.4) (layers "F.Cu" "B.Cu") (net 8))
 (segment (start 134.25 95.5) (end 134.5 95.25) (width 0.2) (layer "B.Cu") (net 8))
 (segment (start 125.5 90.5) (end 125.5 88.9) (width 0.2) (layer "B.Cu") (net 8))
 (segment (start 124.5 95) (end 124.5 90.75) (width 0.2) (layer "B.Cu") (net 8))
 (segment (start 124.5 90.75) (end 124.75 90.5) (width 0.2) (layer "B.Cu") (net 8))
 (segment (start 125.5 91.95) (end 125.5 90.5) (width 0.2) (layer "B.Cu") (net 8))
 (segment (start 125 95.5) (end 124.5 95) (width 0.2) (layer "B.Cu") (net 8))
 (segment (start 129.25 95.5) (end 125 95.5) (width 0.2) (layer "B.Cu") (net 8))
 (segment (start 124.75 90.5) (end 125.5 90.5) (width 0.2) (layer "B.Cu") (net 8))
 (segment (start 129.25 95.5) (end 134.25 95.5) (width 0.2) (layer "B.Cu") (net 8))
 (segment (start 134.635 94.115) (end 134.5 94.25) (width 0.2) (layer "F.Cu") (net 7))
 (segment (start 134.885 94.115) (end 136.2322 94.115) (width 0.2) (layer "F.Cu") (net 7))
 (segment (start 136.2322 94.115) (end 134.635 94.115) (width 0.2) (layer "F.Cu") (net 7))
 (via (at 134.5 94.25) (size 0.8) (drill 0.4) (layers "F.Cu" "B.Cu") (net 7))
 (segment (start 130.25 94.25) (end 130 94) (width 0.2) (layer "B.Cu") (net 7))
 (segment (start 128.5 90.5) (end 128.75 90.75) (width 0.2) (layer "B.Cu") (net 7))
 (segment (start 129.5 93.5) (end 128.75 92.75) (width 0.2) (layer "B.Cu") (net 7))
 (segment (start 127.75 90.5) (end 128.5 90.5) (width 0.2) (layer "B.Cu") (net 7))
 (segment (start 127.75 89.75) (end 127.75 90.5) (width 0.2) (layer "B.Cu") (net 7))
 (segment (start 130 94) (end 129.5 93.5) (width 0.2) (layer "B.Cu") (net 7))
 (segment (start 128.75 92.75) (end 128.75 90.75) (width 0.2) (layer "B.Cu") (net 7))
 (segment (start 127.75 90.5) (end 127.75 91.95) (width 0.2) (layer "B.Cu") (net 7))
 (segment (start 134.5 94.25) (end 130.25 94.25) (width 0.2) (layer "B.Cu") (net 7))
 (segment (start 127.75 86.8) (end 127.75 89.75) (width 0.2) (layer "B.Cu") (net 7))
 (segment (start 134.905 92.845) (end 134.5 93.25) (width 0.2) (layer "F.Cu") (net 6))
 (segment (start 136.2322 92.845) (end 134.905 92.845) (width 0.2) (layer "F.Cu") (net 6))
 (via (at 134.5 93.25) (size 0.8) (drill 0.4) (layers "F.Cu" "B.Cu") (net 6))
 (segment (start 136.75 93) (end 136.75 92.75) (width 0.2) (layer "B.Cu") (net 6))
 (segment (start 136.5 91.75) (end 136.75 92) (width 0.2) (layer "B.Cu") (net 6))
 (segment (start 136.5 93.25) (end 136.75 93) (width 0.2) (layer "B.Cu") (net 6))
 (segment (start 134.5 93.25) (end 136.5 93.25) (width 0.2) (layer "B.Cu") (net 6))
 (segment (start 135.55 91.75) (end 136.5 91.75) (width 0.2) (layer "B.Cu") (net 6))
 (segment (start 136.75 92.5) (end 136.75 92) (width 0.2) (layer "B.Cu") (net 6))
 (segment (start 136.75 92.75) (end 136.75 92.5) (width 0.2) (layer "B.Cu") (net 6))
 (segment (start 134.2 90.5) (end 132 90.5) (width 0.2) (layer "F.Cu") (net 4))
 (via (at 132 90.5) (size 0.8) (drill 0.4) (layers "F.Cu" "B.Cu") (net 4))
 (segment (start 133.25 91.75) (end 132 90.5) (width 0.2) (layer "B.Cu") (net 4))
 (segment (start 133.95 91.75) (end 133.25 91.75) (width 0.2) (layer "B.Cu") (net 4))
 (segment (start 141 89.5) (end 141.25 89.25) (width 0.2) (layer "F.Cu") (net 1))
 (segment (start 140.5 89.75) (end 140.75 89.5) (width 0.2) (layer "F.Cu") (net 1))
 (segment (start 138 89) (end 140 89) (width 0.2) (layer "F.Cu") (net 1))
 (segment (start 140.5 89.5) (end 140.75 89.5) (width 0.2) (layer "F.Cu") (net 1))
 (segment (start 140.75 89.5) (end 141 89.5) (width 0.2) (layer "F.Cu") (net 1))
 (segment (start 140 89) (end 140.5 89.5) (width 0.2) (layer "F.Cu") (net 1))
 (segment (start 140.5 89.75) (end 140.5 89.5) (width 0.2) (layer "F.Cu") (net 1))
 (segment (start 141.45 90.75) (end 140.75 90.75) (width 0.2) (layer "F.Cu") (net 1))
 (segment (start 141.25 89.25) (end 141.25 89) (width 0.2) (layer "F.Cu") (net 1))
 (segment (start 140.5 90.5) (end 140.5 90.25) (width 0.2) (layer "F.Cu") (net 1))
 (segment (start 140.75 90.75) (end 140.5 90.5) (width 0.2) (layer "F.Cu") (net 1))
 (segment (start 140.5 90.25) (end 140.5 89.75) (width 0.2) (layer "F.Cu") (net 1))
 (via (at 138 89) (size 0.8) (drill 0.4) (layers "F.Cu" "B.Cu") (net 1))
 (segment (start 138.25 89.25) (end 138 89) (width 0.2) (layer "B.Cu") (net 1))
 (segment (start 139.6 89.25) (end 138.25 89.25) (width 0.2) (layer "B.Cu") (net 1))
 (segment (start 143.4 89.25) (end 144.25 89.25) (width 0.2) (layer "B.Cu") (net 14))
 (segment (start 144.5 91.75) (end 144.5 91.5) (width 0.2) (layer "B.Cu") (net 14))
 (segment (start 144.25 92) (end 144.5 91.75) (width 0.2) (layer "B.Cu") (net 14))
 (segment (start 144.5 90.5) (end 144.5 91.5) (width 0.2) (layer "B.Cu") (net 14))
 (segment (start 144.25 89.25) (end 144.5 89.5) (width 0.2) (layer "B.Cu") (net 14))
 (segment (start 144.5 90.5) (end 144.5 89.5) (width 0.2) (layer "B.Cu") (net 14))
 (segment (start 143.3 92) (end 144.25 92) (width 0.2) (layer "B.Cu") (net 14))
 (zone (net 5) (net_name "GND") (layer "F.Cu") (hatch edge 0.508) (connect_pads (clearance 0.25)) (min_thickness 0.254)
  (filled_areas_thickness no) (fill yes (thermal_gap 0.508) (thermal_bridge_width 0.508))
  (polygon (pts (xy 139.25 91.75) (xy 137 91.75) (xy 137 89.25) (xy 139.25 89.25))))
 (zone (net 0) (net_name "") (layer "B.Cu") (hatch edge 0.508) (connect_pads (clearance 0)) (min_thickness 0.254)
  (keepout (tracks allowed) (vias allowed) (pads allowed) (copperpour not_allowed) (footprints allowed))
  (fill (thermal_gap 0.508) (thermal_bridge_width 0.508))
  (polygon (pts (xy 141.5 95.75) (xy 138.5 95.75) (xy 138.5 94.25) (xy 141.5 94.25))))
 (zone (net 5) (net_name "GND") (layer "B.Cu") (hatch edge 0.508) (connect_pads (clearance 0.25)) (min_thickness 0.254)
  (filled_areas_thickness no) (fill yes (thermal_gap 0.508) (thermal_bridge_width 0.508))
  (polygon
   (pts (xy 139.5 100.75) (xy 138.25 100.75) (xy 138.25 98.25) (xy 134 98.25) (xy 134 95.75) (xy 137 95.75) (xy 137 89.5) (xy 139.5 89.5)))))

